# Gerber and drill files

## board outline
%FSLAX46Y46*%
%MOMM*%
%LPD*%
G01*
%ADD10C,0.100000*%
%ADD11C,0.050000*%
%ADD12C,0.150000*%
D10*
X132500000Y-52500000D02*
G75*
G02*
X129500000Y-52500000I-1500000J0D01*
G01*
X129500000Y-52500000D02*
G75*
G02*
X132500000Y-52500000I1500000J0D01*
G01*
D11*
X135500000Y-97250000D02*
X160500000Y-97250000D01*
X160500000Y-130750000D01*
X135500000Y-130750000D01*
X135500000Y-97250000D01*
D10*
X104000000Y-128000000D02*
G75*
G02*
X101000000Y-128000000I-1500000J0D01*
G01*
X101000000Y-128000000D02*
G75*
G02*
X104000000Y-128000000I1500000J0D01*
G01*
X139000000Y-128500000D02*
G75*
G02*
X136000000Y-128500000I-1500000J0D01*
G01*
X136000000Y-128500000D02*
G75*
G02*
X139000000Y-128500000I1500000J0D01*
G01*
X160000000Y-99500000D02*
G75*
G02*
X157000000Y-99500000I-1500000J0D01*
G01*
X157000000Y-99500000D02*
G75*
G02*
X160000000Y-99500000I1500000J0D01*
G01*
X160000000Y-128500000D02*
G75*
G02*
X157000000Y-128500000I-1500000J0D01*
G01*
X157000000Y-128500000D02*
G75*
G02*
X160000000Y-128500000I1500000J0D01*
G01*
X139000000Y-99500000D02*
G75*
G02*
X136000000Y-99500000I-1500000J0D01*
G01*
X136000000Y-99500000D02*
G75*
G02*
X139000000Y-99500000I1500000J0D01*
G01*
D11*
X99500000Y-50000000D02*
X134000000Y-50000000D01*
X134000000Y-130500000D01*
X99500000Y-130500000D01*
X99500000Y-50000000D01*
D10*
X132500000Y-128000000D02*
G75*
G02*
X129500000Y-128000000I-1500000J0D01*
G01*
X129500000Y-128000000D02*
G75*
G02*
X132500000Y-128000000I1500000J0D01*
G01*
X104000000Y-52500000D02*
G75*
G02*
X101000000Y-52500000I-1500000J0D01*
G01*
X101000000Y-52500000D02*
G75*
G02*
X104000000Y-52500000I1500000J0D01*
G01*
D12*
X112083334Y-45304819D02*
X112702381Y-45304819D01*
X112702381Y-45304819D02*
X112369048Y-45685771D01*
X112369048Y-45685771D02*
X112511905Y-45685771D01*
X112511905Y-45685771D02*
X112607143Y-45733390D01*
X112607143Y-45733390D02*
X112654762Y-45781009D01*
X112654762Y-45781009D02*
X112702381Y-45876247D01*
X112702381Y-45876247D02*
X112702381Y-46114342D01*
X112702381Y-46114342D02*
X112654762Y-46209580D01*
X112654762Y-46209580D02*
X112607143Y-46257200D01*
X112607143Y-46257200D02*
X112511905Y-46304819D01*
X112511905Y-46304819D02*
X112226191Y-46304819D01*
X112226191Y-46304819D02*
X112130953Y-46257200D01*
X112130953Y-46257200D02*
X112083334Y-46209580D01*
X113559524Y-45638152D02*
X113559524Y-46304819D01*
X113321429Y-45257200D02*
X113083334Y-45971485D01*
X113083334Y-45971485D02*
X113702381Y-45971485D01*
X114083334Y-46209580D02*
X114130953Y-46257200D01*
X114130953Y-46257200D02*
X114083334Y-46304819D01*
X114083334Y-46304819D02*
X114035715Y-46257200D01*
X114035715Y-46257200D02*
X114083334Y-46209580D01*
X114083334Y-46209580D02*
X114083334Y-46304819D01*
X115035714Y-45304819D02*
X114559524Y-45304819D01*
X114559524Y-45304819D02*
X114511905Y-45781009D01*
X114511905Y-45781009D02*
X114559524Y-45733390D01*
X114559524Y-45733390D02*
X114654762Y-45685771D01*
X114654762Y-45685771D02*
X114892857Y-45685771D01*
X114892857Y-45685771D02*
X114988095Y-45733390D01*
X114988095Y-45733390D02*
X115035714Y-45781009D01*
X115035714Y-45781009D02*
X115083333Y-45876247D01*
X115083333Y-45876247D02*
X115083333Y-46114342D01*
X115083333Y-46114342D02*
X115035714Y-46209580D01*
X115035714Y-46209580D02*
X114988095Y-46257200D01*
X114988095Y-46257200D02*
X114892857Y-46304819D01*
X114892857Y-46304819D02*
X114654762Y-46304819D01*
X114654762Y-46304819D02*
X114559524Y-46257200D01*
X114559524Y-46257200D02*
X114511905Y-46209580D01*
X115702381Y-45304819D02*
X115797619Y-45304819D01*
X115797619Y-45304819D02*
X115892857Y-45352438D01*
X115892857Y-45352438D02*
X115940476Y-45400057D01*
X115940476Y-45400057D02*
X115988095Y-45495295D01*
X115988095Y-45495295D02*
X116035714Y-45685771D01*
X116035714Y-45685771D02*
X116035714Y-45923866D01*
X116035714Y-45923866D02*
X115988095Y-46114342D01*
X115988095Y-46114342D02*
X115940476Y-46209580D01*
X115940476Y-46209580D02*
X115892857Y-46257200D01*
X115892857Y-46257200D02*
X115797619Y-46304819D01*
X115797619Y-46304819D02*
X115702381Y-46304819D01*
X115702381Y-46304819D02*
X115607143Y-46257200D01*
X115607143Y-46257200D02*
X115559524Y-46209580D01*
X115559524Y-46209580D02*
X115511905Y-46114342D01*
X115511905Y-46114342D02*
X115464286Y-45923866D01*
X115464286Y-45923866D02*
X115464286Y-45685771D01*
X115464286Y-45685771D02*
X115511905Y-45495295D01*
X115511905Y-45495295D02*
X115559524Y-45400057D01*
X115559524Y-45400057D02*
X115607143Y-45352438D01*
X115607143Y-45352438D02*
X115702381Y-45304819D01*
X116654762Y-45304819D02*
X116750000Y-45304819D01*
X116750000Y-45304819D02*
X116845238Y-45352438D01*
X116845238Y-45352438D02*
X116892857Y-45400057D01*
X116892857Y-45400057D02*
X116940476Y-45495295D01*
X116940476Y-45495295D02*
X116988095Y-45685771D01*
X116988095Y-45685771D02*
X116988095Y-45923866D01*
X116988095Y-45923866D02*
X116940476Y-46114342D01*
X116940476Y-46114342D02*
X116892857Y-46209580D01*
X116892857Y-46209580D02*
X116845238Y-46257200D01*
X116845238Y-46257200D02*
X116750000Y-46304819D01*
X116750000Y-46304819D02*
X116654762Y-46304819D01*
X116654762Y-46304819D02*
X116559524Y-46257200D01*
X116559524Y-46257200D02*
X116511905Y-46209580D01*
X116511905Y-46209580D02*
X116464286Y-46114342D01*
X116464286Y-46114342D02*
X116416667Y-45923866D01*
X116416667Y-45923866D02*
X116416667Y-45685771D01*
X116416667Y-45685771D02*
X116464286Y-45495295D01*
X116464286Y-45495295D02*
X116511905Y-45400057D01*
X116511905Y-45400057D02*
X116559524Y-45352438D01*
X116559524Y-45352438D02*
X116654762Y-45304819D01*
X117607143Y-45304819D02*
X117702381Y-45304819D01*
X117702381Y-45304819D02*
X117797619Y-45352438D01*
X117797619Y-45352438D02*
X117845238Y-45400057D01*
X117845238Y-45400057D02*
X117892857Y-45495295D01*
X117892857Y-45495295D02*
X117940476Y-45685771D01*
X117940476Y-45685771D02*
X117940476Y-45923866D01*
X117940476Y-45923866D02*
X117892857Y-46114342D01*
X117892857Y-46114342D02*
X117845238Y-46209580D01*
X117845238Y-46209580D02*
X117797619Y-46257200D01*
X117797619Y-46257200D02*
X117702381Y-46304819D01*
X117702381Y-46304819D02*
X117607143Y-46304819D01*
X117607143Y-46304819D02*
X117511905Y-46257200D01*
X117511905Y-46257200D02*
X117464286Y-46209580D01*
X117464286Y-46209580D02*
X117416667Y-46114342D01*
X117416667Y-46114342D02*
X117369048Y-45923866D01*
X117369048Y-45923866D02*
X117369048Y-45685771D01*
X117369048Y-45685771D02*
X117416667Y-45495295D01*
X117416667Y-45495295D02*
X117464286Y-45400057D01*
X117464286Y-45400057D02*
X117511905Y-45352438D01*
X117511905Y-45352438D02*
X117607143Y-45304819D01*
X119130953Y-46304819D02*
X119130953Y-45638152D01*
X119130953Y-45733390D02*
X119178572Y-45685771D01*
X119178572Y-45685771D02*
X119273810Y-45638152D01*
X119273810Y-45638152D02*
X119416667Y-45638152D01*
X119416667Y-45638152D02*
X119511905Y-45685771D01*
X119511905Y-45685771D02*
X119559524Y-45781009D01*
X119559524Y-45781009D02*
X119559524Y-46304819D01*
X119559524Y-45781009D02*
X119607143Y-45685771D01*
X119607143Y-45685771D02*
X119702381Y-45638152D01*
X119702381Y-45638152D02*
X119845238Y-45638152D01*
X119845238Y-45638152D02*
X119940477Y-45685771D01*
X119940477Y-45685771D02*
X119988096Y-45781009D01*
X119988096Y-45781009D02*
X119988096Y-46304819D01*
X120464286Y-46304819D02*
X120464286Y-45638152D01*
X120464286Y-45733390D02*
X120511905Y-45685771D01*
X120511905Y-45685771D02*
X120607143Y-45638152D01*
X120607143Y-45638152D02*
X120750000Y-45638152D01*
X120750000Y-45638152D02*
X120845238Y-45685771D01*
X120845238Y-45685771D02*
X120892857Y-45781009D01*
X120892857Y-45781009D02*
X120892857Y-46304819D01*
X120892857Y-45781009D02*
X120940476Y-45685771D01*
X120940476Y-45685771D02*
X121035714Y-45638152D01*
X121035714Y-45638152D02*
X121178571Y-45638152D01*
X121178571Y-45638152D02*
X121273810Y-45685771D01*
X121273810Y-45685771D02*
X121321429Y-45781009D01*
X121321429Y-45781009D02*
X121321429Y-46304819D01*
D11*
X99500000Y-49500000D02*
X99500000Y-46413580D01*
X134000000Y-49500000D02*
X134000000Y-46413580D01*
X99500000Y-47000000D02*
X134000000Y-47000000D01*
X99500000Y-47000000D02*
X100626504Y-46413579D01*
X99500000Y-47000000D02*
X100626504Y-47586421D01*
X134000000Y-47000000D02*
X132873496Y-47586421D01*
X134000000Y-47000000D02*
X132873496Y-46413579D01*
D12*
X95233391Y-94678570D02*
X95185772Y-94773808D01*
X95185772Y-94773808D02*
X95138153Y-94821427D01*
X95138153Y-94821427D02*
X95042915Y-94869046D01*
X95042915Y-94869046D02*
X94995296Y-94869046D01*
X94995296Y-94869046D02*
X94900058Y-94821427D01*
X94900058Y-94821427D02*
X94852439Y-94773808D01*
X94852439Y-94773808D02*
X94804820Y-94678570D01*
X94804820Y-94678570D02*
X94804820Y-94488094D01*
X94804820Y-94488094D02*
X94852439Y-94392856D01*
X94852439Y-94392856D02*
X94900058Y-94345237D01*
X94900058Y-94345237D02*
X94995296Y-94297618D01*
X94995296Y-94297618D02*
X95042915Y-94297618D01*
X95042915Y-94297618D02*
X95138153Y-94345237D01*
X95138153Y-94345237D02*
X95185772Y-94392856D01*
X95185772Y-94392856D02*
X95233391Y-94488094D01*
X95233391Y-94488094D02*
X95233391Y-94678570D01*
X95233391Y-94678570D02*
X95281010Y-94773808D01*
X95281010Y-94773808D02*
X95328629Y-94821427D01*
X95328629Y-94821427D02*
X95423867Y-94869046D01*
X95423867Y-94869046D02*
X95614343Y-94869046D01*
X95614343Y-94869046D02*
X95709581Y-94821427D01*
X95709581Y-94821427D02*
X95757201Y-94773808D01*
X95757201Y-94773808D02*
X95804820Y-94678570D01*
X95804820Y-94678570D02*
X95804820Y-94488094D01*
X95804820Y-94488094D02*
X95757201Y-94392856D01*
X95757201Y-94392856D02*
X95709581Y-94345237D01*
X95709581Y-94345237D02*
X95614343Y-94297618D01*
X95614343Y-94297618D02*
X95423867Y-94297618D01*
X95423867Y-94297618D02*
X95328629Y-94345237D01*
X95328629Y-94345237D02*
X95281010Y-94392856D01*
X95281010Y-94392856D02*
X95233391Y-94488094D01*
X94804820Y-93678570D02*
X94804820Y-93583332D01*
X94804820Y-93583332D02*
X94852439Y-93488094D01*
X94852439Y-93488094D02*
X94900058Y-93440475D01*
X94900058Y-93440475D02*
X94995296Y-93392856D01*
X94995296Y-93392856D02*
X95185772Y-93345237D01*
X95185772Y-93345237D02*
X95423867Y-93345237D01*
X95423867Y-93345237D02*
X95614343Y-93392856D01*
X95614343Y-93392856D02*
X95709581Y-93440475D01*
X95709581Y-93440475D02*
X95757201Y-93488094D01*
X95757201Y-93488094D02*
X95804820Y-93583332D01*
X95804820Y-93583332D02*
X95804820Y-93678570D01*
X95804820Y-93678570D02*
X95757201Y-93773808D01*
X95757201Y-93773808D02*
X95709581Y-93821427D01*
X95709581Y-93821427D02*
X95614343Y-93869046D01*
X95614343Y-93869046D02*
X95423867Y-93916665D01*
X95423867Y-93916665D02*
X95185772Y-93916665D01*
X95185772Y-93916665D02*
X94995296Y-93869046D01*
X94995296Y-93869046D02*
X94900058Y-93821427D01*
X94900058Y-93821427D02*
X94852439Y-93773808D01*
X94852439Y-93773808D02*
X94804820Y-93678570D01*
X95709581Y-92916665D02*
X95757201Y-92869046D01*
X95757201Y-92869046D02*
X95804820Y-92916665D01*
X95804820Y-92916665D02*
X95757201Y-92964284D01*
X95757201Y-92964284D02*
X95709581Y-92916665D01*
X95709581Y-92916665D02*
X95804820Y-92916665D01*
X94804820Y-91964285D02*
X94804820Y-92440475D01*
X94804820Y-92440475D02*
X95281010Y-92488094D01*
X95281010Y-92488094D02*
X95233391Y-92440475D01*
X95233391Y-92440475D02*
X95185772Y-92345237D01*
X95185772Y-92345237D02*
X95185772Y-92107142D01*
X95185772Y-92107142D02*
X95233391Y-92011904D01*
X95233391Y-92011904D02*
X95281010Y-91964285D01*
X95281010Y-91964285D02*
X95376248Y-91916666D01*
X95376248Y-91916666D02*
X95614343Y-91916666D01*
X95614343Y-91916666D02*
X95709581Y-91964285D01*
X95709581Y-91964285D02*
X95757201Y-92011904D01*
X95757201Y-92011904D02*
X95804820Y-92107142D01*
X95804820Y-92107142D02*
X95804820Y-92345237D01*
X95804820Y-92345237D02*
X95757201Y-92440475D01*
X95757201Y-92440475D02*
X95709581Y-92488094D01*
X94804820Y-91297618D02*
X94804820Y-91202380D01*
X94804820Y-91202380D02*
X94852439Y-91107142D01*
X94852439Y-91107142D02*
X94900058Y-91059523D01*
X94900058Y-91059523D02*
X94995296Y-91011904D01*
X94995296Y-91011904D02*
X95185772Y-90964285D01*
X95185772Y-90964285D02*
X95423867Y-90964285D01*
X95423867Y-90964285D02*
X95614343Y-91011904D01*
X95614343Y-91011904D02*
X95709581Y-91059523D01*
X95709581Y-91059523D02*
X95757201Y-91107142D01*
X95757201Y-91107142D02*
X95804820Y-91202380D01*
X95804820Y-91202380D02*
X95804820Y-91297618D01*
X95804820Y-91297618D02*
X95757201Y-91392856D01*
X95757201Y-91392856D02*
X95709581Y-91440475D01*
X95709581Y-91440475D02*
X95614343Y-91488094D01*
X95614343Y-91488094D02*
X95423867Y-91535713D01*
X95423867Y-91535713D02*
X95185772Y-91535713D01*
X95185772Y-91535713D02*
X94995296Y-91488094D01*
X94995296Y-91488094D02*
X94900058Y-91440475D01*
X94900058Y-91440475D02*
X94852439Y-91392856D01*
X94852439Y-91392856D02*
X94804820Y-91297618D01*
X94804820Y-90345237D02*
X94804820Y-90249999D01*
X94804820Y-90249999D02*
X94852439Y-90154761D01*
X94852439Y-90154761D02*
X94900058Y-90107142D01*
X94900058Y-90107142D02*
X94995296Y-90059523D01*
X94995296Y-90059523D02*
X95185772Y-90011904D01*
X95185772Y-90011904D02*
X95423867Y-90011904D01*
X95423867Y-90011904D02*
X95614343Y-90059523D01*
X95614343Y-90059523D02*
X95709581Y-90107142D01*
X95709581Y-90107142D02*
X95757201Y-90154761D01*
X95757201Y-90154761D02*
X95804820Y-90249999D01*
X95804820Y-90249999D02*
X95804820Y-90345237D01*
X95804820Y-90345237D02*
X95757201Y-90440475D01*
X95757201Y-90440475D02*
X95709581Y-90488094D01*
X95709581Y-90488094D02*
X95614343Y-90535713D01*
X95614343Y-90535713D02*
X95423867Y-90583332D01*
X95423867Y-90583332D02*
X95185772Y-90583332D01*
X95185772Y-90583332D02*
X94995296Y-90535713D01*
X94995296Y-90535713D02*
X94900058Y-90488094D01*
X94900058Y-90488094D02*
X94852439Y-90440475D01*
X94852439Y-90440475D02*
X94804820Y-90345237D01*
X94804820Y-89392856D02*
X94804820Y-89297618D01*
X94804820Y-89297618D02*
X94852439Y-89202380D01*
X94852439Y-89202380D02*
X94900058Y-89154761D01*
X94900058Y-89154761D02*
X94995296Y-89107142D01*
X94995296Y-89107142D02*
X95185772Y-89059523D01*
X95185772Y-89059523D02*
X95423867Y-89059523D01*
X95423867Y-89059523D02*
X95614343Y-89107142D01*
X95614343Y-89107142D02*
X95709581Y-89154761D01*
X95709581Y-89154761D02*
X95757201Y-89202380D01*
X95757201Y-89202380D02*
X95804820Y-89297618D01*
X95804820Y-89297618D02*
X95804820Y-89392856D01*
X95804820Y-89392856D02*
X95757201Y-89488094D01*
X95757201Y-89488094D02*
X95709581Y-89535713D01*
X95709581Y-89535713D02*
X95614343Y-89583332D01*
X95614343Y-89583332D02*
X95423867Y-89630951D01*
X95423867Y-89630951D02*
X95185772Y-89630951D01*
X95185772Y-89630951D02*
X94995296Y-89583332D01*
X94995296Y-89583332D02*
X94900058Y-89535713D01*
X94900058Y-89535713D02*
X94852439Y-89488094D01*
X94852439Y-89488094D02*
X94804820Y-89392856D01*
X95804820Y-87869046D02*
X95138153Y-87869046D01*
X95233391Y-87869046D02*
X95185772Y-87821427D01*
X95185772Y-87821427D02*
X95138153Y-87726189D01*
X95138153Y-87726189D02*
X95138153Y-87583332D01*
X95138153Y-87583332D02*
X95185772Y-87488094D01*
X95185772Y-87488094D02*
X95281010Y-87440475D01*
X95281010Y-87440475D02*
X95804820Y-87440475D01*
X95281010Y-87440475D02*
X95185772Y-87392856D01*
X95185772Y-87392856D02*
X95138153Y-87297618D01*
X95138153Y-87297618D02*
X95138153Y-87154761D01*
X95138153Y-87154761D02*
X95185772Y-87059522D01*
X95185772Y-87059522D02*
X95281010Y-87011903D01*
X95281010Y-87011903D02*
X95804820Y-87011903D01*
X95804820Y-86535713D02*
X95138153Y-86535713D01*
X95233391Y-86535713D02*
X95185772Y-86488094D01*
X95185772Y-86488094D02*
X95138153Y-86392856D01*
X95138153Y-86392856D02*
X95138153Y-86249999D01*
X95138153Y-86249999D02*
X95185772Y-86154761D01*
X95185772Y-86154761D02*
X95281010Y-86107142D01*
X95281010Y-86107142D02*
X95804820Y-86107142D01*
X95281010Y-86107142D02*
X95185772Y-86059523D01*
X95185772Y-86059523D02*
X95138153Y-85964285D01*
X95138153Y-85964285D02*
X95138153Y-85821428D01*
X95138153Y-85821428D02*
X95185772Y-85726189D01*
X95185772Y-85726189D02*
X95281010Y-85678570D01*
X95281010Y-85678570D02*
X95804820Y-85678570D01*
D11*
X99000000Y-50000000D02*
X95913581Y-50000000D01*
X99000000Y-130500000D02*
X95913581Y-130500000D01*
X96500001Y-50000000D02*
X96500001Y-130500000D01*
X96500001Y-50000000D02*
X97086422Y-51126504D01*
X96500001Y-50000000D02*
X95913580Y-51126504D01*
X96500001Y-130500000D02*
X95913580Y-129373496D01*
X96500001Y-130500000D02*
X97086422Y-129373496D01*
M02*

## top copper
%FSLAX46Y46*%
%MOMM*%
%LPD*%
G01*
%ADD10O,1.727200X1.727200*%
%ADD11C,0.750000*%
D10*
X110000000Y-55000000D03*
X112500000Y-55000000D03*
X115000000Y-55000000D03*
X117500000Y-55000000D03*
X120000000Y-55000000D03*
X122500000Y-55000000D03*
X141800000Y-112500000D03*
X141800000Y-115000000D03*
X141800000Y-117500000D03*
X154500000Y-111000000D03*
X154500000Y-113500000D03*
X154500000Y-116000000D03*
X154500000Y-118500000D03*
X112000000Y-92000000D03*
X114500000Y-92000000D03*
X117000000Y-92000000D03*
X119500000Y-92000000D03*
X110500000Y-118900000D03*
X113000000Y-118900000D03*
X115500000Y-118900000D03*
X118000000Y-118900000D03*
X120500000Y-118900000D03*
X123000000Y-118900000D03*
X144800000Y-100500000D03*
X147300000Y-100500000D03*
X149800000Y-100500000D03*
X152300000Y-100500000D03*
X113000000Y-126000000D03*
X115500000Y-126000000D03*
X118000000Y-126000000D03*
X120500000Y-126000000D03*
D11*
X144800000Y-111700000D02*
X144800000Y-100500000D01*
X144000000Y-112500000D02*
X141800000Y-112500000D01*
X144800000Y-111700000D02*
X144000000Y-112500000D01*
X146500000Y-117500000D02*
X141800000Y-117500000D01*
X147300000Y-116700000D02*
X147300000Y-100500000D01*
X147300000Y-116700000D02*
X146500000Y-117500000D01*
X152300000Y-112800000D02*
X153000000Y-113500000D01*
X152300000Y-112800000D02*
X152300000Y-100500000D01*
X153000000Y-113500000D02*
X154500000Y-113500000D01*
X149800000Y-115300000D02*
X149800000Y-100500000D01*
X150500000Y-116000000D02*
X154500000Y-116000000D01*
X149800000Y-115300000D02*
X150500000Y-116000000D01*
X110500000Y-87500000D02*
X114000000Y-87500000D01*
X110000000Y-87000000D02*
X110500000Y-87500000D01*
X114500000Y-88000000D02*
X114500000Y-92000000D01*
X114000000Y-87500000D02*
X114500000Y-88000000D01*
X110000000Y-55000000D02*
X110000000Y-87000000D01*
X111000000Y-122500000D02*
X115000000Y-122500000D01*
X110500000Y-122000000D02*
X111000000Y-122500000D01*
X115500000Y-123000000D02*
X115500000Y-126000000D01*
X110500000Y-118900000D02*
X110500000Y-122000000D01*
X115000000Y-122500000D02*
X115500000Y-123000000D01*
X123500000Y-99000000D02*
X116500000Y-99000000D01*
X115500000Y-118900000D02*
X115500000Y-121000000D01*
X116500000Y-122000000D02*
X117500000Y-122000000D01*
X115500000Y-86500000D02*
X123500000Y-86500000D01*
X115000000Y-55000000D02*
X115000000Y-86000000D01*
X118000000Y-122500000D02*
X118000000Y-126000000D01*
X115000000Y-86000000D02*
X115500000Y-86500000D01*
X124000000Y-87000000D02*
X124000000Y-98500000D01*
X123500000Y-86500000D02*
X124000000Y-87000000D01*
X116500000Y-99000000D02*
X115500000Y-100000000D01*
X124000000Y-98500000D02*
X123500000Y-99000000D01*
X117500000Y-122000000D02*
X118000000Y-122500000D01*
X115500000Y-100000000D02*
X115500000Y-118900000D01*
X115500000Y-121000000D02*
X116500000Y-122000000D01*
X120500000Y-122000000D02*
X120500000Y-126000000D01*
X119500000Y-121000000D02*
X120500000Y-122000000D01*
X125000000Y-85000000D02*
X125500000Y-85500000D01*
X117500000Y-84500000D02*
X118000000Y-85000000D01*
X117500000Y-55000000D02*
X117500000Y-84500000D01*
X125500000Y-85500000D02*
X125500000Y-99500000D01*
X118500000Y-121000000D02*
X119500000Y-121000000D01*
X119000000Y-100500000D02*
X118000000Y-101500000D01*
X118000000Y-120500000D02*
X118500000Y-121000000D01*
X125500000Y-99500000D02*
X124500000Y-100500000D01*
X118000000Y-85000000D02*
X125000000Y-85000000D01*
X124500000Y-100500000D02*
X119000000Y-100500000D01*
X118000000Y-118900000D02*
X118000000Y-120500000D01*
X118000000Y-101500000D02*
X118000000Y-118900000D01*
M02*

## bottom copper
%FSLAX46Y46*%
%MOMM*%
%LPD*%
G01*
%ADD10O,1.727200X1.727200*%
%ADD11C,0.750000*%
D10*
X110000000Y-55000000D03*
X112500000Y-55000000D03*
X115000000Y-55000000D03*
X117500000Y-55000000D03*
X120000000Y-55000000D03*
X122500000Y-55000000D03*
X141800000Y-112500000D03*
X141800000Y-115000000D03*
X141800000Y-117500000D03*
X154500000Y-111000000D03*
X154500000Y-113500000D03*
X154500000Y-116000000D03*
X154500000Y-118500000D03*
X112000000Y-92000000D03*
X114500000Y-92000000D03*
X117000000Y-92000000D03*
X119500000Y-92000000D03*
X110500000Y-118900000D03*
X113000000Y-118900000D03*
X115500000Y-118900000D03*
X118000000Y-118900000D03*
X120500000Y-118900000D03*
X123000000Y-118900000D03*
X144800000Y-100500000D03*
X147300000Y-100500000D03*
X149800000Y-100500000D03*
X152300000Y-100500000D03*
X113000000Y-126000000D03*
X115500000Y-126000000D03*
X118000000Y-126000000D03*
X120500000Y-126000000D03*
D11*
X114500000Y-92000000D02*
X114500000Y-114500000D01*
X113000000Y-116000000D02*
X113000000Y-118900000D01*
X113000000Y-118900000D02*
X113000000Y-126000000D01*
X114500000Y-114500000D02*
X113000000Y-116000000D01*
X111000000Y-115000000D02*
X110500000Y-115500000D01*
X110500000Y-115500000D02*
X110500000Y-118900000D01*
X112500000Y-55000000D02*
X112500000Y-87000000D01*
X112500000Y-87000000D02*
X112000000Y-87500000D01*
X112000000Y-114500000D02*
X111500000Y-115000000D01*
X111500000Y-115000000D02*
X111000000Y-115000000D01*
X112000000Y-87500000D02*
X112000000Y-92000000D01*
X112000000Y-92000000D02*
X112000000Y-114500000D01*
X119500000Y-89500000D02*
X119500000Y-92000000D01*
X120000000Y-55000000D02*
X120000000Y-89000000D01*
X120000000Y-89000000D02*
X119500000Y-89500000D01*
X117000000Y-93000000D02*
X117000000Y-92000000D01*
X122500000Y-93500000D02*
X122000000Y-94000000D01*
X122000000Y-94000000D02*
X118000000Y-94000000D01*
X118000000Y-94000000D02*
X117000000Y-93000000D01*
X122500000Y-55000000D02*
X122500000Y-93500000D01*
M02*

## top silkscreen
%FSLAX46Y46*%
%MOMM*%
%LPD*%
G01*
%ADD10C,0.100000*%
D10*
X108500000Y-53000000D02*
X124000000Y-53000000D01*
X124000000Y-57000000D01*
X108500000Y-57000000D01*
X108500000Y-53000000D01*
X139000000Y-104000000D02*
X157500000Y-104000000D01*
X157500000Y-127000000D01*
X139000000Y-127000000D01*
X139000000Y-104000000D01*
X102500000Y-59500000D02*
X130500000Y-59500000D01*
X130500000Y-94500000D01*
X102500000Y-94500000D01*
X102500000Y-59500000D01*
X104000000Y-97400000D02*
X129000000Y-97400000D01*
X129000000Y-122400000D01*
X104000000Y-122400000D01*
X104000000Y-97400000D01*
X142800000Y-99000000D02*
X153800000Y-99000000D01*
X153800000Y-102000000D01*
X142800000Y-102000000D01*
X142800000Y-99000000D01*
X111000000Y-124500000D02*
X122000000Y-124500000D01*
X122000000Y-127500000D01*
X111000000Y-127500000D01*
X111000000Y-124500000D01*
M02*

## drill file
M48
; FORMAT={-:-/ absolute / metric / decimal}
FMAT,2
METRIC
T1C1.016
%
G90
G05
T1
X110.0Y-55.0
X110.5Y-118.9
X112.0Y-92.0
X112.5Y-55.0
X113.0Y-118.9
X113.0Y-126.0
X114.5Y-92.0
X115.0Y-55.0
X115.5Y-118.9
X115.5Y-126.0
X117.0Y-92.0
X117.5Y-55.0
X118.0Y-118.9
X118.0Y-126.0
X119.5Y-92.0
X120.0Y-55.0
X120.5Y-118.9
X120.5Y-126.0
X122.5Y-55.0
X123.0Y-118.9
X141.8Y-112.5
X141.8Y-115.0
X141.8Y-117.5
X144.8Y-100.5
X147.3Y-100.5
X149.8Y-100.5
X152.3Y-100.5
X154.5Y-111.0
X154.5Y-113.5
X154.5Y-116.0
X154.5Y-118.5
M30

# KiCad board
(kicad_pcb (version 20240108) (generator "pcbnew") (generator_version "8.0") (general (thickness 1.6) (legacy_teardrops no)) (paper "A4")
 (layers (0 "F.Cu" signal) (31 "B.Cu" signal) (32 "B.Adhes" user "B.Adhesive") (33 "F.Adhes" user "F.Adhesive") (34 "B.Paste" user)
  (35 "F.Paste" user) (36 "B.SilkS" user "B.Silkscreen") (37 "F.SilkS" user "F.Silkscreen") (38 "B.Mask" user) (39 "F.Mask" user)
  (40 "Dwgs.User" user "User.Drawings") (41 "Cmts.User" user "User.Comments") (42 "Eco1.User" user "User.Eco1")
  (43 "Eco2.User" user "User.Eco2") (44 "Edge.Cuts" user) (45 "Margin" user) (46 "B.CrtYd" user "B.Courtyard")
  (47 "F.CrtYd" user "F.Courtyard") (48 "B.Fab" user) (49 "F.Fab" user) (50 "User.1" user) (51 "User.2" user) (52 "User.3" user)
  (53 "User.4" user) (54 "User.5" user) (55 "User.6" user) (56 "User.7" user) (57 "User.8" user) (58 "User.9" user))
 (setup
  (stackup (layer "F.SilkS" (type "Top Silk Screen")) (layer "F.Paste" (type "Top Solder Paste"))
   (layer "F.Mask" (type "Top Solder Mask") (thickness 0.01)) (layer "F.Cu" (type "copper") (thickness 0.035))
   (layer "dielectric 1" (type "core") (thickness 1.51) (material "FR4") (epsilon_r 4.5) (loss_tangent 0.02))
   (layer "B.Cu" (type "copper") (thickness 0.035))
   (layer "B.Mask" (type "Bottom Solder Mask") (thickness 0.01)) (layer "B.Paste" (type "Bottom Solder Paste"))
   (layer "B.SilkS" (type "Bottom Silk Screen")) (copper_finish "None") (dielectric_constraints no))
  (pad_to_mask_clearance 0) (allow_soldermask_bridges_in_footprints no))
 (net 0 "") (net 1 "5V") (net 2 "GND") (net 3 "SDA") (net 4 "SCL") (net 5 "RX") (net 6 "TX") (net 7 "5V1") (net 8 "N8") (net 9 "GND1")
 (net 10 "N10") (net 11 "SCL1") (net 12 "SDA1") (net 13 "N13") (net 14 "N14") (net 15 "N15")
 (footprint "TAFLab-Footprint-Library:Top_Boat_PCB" (layer "F.Cu") (at 115 60)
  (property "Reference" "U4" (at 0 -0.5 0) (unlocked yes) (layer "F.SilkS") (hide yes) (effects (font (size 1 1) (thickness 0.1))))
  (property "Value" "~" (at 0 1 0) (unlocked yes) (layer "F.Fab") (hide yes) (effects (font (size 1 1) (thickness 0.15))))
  (fp_rect (start -6.5 -7) (end 9 -3) (stroke (width 0.1) (type default)) (fill none) (layer "F.SilkS"))
  (pad "1" thru_hole oval (at -5 -5) (size 1.7272 1.7272) (drill 1.016) (layers "*.Cu" "*.Mask") (remove_unused_layers no) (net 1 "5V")
   (thermal_bridge_angle 45))
  (pad "2" thru_hole oval (at -2.5 -5) (size 1.7272 1.7272) (drill 1.016) (layers "*.Cu" "*.Mask") (remove_unused_layers no) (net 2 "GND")
   (thermal_bridge_angle 45))
  (pad "3" thru_hole oval (at 0 -5) (size 1.7272 1.7272) (drill 1.016) (layers "*.Cu" "*.Mask") (remove_unused_layers no) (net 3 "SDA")
   (thermal_bridge_angle 45))
  (pad "4" thru_hole oval (at 2.5 -5) (size 1.7272 1.7272) (drill 1.016) (layers "*.Cu" "*.Mask") (remove_unused_layers no) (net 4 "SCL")
   (thermal_bridge_angle 45))
  (pad "5" thru_hole oval (at 5 -5) (size 1.7272 1.7272) (drill 1.016) (layers "*.Cu" "*.Mask") (remove_unused_layers no) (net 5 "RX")
   (thermal_bridge_angle 45))
  (pad "6" thru_hole oval (at 7.5 -5) (size 1.7272 1.7272) (drill 1.016) (layers "*.Cu" "*.Mask") (remove_unused_layers no) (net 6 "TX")
   (thermal_bridge_angle 45)))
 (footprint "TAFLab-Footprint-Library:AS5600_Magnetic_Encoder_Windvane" (layer "F.Cu") (at 135.5 122.5)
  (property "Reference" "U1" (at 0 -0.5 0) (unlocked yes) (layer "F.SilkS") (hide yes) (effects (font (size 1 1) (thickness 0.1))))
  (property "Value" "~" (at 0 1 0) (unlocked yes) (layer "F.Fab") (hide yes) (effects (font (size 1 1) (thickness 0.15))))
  (fp_rect (start 3.5 -18.5) (end 22 4.5) (stroke (width 0.1) (type default)) (fill none) (layer "F.SilkS"))
  (pad "1" thru_hole oval (at 6.3 -10) (size 1.7272 1.7272) (drill 1.016) (layers "*.Cu" "*.Mask") (remove_unused_layers no) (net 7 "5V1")
   (thermal_bridge_angle 45))
  (pad "2" thru_hole oval (at 6.3 -7.5) (size 1.7272 1.7272) (drill 1.016) (layers "*.Cu" "*.Mask") (remove_unused_layers no) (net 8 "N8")
   (thermal_bridge_angle 45))
  (pad "3" thru_hole oval (at 6.3 -5) (size 1.7272 1.7272) (drill 1.016) (layers "*.Cu" "*.Mask") (remove_unused_layers no) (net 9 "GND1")
   (thermal_bridge_angle 45))
  (pad "4" thru_hole oval (at 19 -11.5) (size 1.7272 1.7272) (drill 1.016) (layers "*.Cu" "*.Mask") (remove_unused_layers no) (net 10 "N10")
   (thermal_bridge_angle 45))
  (pad "5" thru_hole oval (at 19 -9) (size 1.7272 1.7272) (drill 1.016) (layers "*.Cu" "*.Mask") (remove_unused_layers no) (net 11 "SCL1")
   (thermal_bridge_angle 45))
  (pad "6" thru_hole oval (at 19 -6.5) (size 1.7272 1.7272) (drill 1.016) (layers "*.Cu" "*.Mask") (remove_unused_layers no) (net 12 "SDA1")
   (thermal_bridge_angle 45))
  (pad "7" thru_hole oval (at 19 -4) (size 1.7272 1.7272) (drill 1.016) (layers "*.Cu" "*.Mask") (remove_unused_layers no) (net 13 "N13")
   (thermal_bridge_angle 45)))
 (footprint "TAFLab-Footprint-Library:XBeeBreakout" (layer "F.Cu") (at 122 92 90)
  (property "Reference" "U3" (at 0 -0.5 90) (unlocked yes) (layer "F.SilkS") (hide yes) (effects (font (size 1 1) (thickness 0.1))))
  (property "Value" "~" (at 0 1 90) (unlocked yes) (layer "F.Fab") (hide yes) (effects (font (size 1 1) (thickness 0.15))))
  (fp_rect (start -2.5 -19.5) (end 32.5 8.5) (stroke (width 0.1) (type default)) (fill none) (layer "F.SilkS"))
  (pad "1" thru_hole oval (at 0 -10 90) (size 1.7272 1.7272) (drill 1.016) (layers "*.Cu" "*.Mask") (remove_unused_layers no) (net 2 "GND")
   (thermal_bridge_angle 45))
  (pad "2" thru_hole oval (at 0 -7.5 90) (size 1.7272 1.7272) (drill 1.016) (layers "*.Cu" "*.Mask") (remove_unused_layers no) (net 1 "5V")
   (thermal_bridge_angle 45))
  (pad "3" thru_hole oval (at 0 -5 90) (size 1.7272 1.7272) (drill 1.016) (layers "*.Cu" "*.Mask") (remove_unused_layers no) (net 6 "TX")
   (thermal_bridge_angle 45))
  (pad "4" thru_hole oval (at 0 -2.5 90) (size 1.7272 1.7272) (drill 1.016) (layers "*.Cu" "*.Mask") (remove_unused_layers no) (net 5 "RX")
   (thermal_bridge_angle 45)))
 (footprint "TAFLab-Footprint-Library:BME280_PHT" (layer "F.Cu") (at 120.5 132.4 90)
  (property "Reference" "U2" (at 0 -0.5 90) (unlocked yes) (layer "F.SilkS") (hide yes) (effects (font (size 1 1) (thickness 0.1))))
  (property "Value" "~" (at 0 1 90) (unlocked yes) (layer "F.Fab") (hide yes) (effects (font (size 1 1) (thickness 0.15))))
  (fp_rect (start 10 -16.5) (end 35 8.5) (stroke (width 0.1) (type default)) (fill none) (layer "F.SilkS"))
  (pad "1" thru_hole oval (at 13.5 -10 90) (size 1.7272 1.7272) (drill 1.016) (layers "*.Cu" "*.Mask") (remove_unused_layers no)
   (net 2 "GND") (thermal_bridge_angle 45))
  (pad "2" thru_hole oval (at 13.5 -7.5 90) (size 1.7272 1.7272) (drill 1.016) (layers "*.Cu" "*.Mask") (remove_unused_layers no)
   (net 1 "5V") (thermal_bridge_angle 45))
  (pad "3" thru_hole oval (at 13.5 -5 90) (size 1.7272 1.7272) (drill 1.016) (layers "*.Cu" "*.Mask") (remove_unused_layers no)
   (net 3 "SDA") (thermal_bridge_angle 45))
  (pad "4" thru_hole oval (at 13.5 -2.5 90) (size 1.7272 1.7272) (drill 1.016) (layers "*.Cu" "*.Mask") (remove_unused_layers no)
   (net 4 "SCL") (thermal_bridge_angle 45))
  (pad "5" thru_hole oval (at 13.5 0 90) (size 1.7272 1.7272) (drill 1.016) (layers "*.Cu" "*.Mask") (remove_unused_layers no)
   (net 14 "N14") (thermal_bridge_angle 45))
  (pad "6" thru_hole oval (at 13.5 2.5 90) (size 1.7272 1.7272) (drill 1.016) (layers "*.Cu" "*.Mask") (remove_unused_layers no)
   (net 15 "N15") (thermal_bridge_angle 45)))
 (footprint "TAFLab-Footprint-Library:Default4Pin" (layer "F.Cu") (at 159.8 100.5 90)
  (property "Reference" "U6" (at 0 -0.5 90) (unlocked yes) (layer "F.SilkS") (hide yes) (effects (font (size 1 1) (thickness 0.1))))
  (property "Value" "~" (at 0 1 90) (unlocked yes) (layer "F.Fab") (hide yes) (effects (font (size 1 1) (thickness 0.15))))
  (fp_rect (start -1.5 -17) (end 1.5 -6) (stroke (width 0.1) (type default)) (fill none) (layer "F.SilkS"))
  (pad "1" thru_hole oval (at 0 -15 90) (size 1.7272 1.7272) (drill 1.016) (layers "*.Cu" "*.Mask") (remove_unused_layers no) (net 7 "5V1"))
  (pad "2" thru_hole oval (at 0 -12.5 90) (size 1.7272 1.7272) (drill 1.016) (layers "*.Cu" "*.Mask") (remove_unused_layers no)
   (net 9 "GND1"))
  (pad "3" thru_hole oval (at 0 -10 90) (size 1.7272 1.7272) (drill 1.016) (layers "*.Cu" "*.Mask") (remove_unused_layers no)
   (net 12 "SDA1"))
  (pad "4" thru_hole oval (at 0 -7.5 90) (size 1.7272 1.7272) (drill 1.016) (layers "*.Cu" "*.Mask") (remove_unused_layers no)
   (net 11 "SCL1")))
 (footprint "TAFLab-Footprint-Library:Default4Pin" (layer "F.Cu") (at 128 126 90)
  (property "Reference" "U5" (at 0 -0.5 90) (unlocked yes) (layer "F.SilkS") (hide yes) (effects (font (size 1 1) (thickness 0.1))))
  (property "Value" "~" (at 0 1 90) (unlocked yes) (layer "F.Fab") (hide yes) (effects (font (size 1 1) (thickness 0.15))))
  (fp_rect (start -1.5 -17) (end 1.5 -6) (stroke (width 0.1) (type default)) (fill none) (layer "F.SilkS"))
  (pad "1" thru_hole oval (at 0 -15 90) (size 1.7272 1.7272) (drill 1.016) (layers "*.Cu" "*.Mask") (remove_unused_layers no) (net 1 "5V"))
  (pad "2" thru_hole oval (at 0 -12.5 90) (size 1.7272 1.7272) (drill 1.016) (layers "*.Cu" "*.Mask") (remove_unused_layers no)
   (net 2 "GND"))
  (pad "3" thru_hole oval (at 0 -10 90) (size 1.7272 1.7272) (drill 1.016) (layers "*.Cu" "*.Mask") (remove_unused_layers no) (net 3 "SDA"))
  (pad "4" thru_hole oval (at 0 -7.5 90) (size 1.7272 1.7272) (drill 1.016) (layers "*.Cu" "*.Mask") (remove_unused_layers no) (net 4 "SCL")))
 (gr_circle (center 131 52.5) (end 132.5 52.5) (stroke (width 0.1) (type default)) (fill none) (layer "Edge.Cuts"))
 (gr_rect (start 135.5 97.25) (end 160.5 130.75) (stroke (width 0.05) (type default)) (fill none) (layer "Edge.Cuts"))
 (gr_circle (center 102.5 128) (end 104 128) (stroke (width 0.1) (type default)) (fill none) (layer "Edge.Cuts"))
 (gr_circle (center 137.5 128.5) (end 139 128.5) (stroke (width 0.1) (type default)) (fill none) (layer "Edge.Cuts"))
 (gr_circle (center 158.5 99.5) (end 160 99.5) (stroke (width 0.1) (type default)) (fill none) (layer "Edge.Cuts"))
 (gr_circle (center 158.5 128.5) (end 160 128.5) (stroke (width 0.1) (type default)) (fill none) (layer "Edge.Cuts"))
 (gr_circle (center 137.5 99.5) (end 139 99.5) (stroke (width 0.1) (type default)) (fill none) (layer "Edge.Cuts"))
 (gr_rect (start 99.5 50) (end 134 130.5) (stroke (width 0.05) (type default)) (fill none) (layer "Edge.Cuts"))
 (gr_circle (center 131 128) (end 132.5 128) (stroke (width 0.1) (type default)) (fill none) (layer "Edge.Cuts"))
 (gr_circle (center 102.5 52.5) (end 104 52.5) (stroke (width 0.1) (type default)) (fill none) (layer "Edge.Cuts"))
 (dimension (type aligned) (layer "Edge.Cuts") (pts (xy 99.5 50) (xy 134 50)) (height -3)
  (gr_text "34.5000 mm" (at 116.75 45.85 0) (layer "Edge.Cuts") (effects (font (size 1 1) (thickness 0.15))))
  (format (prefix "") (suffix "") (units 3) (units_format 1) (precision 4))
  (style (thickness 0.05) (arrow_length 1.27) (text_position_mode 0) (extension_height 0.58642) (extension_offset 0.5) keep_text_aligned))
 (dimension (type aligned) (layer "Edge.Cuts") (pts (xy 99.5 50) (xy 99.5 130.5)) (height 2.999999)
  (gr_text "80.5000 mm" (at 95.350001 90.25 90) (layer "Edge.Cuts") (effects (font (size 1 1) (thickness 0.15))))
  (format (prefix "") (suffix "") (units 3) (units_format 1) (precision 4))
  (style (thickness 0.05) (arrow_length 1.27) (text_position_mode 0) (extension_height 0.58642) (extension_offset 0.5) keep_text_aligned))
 (segment (start 144.8 111.7) (end 144.8 100.5) (width 0.75) (layer "F.Cu") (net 7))
 (segment (start 144 112.5) (end 141.8 112.5) (width 0.75) (layer "F.Cu") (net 7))
 (segment (start 144.8 111.7) (end 144 112.5) (width 0.75) (layer "F.Cu") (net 7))
 (segment (start 146.5 117.5) (end 141.8 117.5) (width 0.75) (layer "F.Cu") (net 9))
 (segment (start 147.3 116.7) (end 147.3 100.5) (width 0.75) (layer "F.Cu") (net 9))
 (segment (start 147.3 116.7) (end 146.5 117.5) (width 0.75) (layer "F.Cu") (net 9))
 (segment (start 152.3 112.8) (end 153 113.5) (width 0.75) (layer "F.Cu") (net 11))
 (segment (start 152.3 112.8) (end 152.3 100.5) (width 0.75) (layer "F.Cu") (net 11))
 (segment (start 153 113.5) (end 154.5 113.5) (width 0.75) (layer "F.Cu") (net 11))
 (segment (start 149.8 115.3) (end 149.8 100.5) (width 0.75) (layer "F.Cu") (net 12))
 (segment (start 150.5 116) (end 154.5 116) (width 0.75) (layer "F.Cu") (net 12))
 (segment (start 149.8 115.3) (end 150.5 116) (width 0.75) (layer "F.Cu") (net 12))
 (segment (start 110.5 87.5) (end 114 87.5) (width 0.75) (layer "F.Cu") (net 1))
 (segment (start 110 87) (end 110.5 87.5) (width 0.75) (layer "F.Cu") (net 1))
 (segment (start 114.5 88) (end 114.5 92) (width 0.75) (layer "F.Cu") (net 1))
 (segment (start 114 87.5) (end 114.5 88) (width 0.75) (layer "F.Cu") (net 1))
 (segment (start 110 55) (end 110 87) (width 0.75) (layer "F.Cu") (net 1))
 (segment (start 114.5 92) (end 114.5 114.5) (width 0.75) (layer "B.Cu") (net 1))
 (segment (start 113 116) (end 113 118.9) (width 0.75) (layer "B.Cu") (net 1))
 (segment (start 113 118.9) (end 113 126) (width 0.75) (layer "B.Cu") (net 1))
 (segment (start 114.5 114.5) (end 113 116) (width 0.75) (layer "B.Cu") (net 1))
 (segment (start 111 122.5) (end 115 122.5) (width 0.75) (layer "F.Cu") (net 2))
 (segment (start 110.5 122) (end 111 122.5) (width 0.75) (layer "F.Cu") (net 2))
 (segment (start 115.5 123) (end 115.5 126) (width 0.75) (layer "F.Cu") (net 2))
 (segment (start 110.5 118.9) (end 110.5 122) (width 0.75) (layer "F.Cu") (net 2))
 (segment (start 115 122.5) (end 115.5 123) (width 0.75) (layer "F.Cu") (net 2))
 (segment (start 111 115) (end 110.5 115.5) (width 0.75) (layer "B.Cu") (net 2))
 (segment (start 110.5 115.5) (end 110.5 118.9) (width 0.75) (layer "B.Cu") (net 2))
 (segment (start 112.5 55) (end 112.5 87) (width 0.75) (layer "B.Cu") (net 2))
 (segment (start 112.5 87) (end 112 87.5) (width 0.75) (layer "B.Cu") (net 2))
 (segment (start 112 114.5) (end 111.5 115) (width 0.75) (layer "B.Cu") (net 2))
 (segment (start 111.5 115) (end 111 115) (width 0.75) (layer "B.Cu") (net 2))
 (segment (start 112 87.5) (end 112 92) (width 0.75) (layer "B.Cu") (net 2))
 (segment (start 112 92) (end 112 114.5) (width 0.75) (layer "B.Cu") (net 2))
 (segment (start 123.5 99) (end 116.5 99) (width 0.75) (layer "F.Cu") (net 3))
 (segment (start 115.5 118.9) (end 115.5 121) (width 0.75) (layer "F.Cu") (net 3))
 (segment (start 116.5 122) (end 117.5 122) (width 0.75) (layer "F.Cu") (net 3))
 (segment (start 115.5 86.5) (end 123.5 86.5) (width 0.75) (layer "F.Cu") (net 3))
 (segment (start 115 55) (end 115 86) (width 0.75) (layer "F.Cu") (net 3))
 (segment (start 118 122.5) (end 118 126) (width 0.75) (layer "F.Cu") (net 3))
 (segment (start 115 86) (end 115.5 86.5) (width 0.75) (layer "F.Cu") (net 3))
 (segment (start 124 87) (end 124 98.5) (width 0.75) (layer "F.Cu") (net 3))
 (segment (start 123.5 86.5) (end 124 87) (width 0.75) (layer "F.Cu") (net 3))
 (segment (start 116.5 99) (end 115.5 100) (width 0.75) (layer "F.Cu") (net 3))
 (segment (start 124 98.5) (end 123.5 99) (width 0.75) (layer "F.Cu") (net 3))
 (segment (start 117.5 122) (end 118 122.5) (width 0.75) (layer "F.Cu") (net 3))
 (segment (start 115.5 100) (end 115.5 118.9) (width 0.75) (layer "F.Cu") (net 3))
 (segment (start 115.5 121) (end 116.5 122) (width 0.75) (layer "F.Cu") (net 3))
 (segment (start 120.5 122) (end 120.5 126) (width 0.75) (layer "F.Cu") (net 4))
 (segment (start 119.5 121) (end 120.5 122) (width 0.75) (layer "F.Cu") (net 4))
 (segment (start 125 85) (end 125.5 85.5) (width 0.75) (layer "F.Cu") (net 4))
 (segment (start 117.5 84.5) (end 118 85) (width 0.75) (layer "F.Cu") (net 4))
 (segment (start 117.5 55) (end 117.5 84.5) (width 0.75) (layer "F.Cu") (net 4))
 (segment (start 125.5 85.5) (end 125.5 99.5) (width 0.75) (layer "F.Cu") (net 4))
 (segment (start 118.5 121) (end 119.5 121) (width 0.75) (layer "F.Cu") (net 4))
 (segment (start 119 100.5) (end 118 101.5) (width 0.75) (layer "F.Cu") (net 4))
 (segment (start 118 120.5) (end 118.5 121) (width 0.75) (layer "F.Cu") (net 4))
 (segment (start 125.5 99.5) (end 124.5 100.5) (width 0.75) (layer "F.Cu") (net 4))
 (segment (start 118 85) (end 125 85) (width 0.75) (layer "F.Cu") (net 4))
 (segment (start 124.5 100.5) (end 119 100.5) (width 0.75) (layer "F.Cu") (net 4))
 (segment (start 118 118.9) (end 118 120.5) (width 0.75) (layer "F.Cu") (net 4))
 (segment (start 118 101.5) (end 118 118.9) (width 0.75) (layer "F.Cu") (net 4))
 (segment (start 119.5 89.5) (end 119.5 92) (width 0.75) (layer "B.Cu") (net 5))
 (segment (start 120 55) (end 120 89) (width 0.75) (layer "B.Cu") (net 5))
 (segment (start 120 89) (end 119.5 89.5) (width 0.75) (layer "B.Cu") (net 5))
 (segment (start 117 93) (end 117 92) (width 0.75) (layer "B.Cu") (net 6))
 (segment (start 122.5 93.5) (end 122 94) (width 0.75) (layer "B.Cu") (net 6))
 (segment (start 122 94) (end 118 94) (width 0.75) (layer "B.Cu") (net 6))
 (segment (start 118 94) (end 117 93) (width 0.75) (layer "B.Cu") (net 6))
 (segment (start 122.5 55) (end 122.5 93.5) (width 0.75) (layer "B.Cu") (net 6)))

